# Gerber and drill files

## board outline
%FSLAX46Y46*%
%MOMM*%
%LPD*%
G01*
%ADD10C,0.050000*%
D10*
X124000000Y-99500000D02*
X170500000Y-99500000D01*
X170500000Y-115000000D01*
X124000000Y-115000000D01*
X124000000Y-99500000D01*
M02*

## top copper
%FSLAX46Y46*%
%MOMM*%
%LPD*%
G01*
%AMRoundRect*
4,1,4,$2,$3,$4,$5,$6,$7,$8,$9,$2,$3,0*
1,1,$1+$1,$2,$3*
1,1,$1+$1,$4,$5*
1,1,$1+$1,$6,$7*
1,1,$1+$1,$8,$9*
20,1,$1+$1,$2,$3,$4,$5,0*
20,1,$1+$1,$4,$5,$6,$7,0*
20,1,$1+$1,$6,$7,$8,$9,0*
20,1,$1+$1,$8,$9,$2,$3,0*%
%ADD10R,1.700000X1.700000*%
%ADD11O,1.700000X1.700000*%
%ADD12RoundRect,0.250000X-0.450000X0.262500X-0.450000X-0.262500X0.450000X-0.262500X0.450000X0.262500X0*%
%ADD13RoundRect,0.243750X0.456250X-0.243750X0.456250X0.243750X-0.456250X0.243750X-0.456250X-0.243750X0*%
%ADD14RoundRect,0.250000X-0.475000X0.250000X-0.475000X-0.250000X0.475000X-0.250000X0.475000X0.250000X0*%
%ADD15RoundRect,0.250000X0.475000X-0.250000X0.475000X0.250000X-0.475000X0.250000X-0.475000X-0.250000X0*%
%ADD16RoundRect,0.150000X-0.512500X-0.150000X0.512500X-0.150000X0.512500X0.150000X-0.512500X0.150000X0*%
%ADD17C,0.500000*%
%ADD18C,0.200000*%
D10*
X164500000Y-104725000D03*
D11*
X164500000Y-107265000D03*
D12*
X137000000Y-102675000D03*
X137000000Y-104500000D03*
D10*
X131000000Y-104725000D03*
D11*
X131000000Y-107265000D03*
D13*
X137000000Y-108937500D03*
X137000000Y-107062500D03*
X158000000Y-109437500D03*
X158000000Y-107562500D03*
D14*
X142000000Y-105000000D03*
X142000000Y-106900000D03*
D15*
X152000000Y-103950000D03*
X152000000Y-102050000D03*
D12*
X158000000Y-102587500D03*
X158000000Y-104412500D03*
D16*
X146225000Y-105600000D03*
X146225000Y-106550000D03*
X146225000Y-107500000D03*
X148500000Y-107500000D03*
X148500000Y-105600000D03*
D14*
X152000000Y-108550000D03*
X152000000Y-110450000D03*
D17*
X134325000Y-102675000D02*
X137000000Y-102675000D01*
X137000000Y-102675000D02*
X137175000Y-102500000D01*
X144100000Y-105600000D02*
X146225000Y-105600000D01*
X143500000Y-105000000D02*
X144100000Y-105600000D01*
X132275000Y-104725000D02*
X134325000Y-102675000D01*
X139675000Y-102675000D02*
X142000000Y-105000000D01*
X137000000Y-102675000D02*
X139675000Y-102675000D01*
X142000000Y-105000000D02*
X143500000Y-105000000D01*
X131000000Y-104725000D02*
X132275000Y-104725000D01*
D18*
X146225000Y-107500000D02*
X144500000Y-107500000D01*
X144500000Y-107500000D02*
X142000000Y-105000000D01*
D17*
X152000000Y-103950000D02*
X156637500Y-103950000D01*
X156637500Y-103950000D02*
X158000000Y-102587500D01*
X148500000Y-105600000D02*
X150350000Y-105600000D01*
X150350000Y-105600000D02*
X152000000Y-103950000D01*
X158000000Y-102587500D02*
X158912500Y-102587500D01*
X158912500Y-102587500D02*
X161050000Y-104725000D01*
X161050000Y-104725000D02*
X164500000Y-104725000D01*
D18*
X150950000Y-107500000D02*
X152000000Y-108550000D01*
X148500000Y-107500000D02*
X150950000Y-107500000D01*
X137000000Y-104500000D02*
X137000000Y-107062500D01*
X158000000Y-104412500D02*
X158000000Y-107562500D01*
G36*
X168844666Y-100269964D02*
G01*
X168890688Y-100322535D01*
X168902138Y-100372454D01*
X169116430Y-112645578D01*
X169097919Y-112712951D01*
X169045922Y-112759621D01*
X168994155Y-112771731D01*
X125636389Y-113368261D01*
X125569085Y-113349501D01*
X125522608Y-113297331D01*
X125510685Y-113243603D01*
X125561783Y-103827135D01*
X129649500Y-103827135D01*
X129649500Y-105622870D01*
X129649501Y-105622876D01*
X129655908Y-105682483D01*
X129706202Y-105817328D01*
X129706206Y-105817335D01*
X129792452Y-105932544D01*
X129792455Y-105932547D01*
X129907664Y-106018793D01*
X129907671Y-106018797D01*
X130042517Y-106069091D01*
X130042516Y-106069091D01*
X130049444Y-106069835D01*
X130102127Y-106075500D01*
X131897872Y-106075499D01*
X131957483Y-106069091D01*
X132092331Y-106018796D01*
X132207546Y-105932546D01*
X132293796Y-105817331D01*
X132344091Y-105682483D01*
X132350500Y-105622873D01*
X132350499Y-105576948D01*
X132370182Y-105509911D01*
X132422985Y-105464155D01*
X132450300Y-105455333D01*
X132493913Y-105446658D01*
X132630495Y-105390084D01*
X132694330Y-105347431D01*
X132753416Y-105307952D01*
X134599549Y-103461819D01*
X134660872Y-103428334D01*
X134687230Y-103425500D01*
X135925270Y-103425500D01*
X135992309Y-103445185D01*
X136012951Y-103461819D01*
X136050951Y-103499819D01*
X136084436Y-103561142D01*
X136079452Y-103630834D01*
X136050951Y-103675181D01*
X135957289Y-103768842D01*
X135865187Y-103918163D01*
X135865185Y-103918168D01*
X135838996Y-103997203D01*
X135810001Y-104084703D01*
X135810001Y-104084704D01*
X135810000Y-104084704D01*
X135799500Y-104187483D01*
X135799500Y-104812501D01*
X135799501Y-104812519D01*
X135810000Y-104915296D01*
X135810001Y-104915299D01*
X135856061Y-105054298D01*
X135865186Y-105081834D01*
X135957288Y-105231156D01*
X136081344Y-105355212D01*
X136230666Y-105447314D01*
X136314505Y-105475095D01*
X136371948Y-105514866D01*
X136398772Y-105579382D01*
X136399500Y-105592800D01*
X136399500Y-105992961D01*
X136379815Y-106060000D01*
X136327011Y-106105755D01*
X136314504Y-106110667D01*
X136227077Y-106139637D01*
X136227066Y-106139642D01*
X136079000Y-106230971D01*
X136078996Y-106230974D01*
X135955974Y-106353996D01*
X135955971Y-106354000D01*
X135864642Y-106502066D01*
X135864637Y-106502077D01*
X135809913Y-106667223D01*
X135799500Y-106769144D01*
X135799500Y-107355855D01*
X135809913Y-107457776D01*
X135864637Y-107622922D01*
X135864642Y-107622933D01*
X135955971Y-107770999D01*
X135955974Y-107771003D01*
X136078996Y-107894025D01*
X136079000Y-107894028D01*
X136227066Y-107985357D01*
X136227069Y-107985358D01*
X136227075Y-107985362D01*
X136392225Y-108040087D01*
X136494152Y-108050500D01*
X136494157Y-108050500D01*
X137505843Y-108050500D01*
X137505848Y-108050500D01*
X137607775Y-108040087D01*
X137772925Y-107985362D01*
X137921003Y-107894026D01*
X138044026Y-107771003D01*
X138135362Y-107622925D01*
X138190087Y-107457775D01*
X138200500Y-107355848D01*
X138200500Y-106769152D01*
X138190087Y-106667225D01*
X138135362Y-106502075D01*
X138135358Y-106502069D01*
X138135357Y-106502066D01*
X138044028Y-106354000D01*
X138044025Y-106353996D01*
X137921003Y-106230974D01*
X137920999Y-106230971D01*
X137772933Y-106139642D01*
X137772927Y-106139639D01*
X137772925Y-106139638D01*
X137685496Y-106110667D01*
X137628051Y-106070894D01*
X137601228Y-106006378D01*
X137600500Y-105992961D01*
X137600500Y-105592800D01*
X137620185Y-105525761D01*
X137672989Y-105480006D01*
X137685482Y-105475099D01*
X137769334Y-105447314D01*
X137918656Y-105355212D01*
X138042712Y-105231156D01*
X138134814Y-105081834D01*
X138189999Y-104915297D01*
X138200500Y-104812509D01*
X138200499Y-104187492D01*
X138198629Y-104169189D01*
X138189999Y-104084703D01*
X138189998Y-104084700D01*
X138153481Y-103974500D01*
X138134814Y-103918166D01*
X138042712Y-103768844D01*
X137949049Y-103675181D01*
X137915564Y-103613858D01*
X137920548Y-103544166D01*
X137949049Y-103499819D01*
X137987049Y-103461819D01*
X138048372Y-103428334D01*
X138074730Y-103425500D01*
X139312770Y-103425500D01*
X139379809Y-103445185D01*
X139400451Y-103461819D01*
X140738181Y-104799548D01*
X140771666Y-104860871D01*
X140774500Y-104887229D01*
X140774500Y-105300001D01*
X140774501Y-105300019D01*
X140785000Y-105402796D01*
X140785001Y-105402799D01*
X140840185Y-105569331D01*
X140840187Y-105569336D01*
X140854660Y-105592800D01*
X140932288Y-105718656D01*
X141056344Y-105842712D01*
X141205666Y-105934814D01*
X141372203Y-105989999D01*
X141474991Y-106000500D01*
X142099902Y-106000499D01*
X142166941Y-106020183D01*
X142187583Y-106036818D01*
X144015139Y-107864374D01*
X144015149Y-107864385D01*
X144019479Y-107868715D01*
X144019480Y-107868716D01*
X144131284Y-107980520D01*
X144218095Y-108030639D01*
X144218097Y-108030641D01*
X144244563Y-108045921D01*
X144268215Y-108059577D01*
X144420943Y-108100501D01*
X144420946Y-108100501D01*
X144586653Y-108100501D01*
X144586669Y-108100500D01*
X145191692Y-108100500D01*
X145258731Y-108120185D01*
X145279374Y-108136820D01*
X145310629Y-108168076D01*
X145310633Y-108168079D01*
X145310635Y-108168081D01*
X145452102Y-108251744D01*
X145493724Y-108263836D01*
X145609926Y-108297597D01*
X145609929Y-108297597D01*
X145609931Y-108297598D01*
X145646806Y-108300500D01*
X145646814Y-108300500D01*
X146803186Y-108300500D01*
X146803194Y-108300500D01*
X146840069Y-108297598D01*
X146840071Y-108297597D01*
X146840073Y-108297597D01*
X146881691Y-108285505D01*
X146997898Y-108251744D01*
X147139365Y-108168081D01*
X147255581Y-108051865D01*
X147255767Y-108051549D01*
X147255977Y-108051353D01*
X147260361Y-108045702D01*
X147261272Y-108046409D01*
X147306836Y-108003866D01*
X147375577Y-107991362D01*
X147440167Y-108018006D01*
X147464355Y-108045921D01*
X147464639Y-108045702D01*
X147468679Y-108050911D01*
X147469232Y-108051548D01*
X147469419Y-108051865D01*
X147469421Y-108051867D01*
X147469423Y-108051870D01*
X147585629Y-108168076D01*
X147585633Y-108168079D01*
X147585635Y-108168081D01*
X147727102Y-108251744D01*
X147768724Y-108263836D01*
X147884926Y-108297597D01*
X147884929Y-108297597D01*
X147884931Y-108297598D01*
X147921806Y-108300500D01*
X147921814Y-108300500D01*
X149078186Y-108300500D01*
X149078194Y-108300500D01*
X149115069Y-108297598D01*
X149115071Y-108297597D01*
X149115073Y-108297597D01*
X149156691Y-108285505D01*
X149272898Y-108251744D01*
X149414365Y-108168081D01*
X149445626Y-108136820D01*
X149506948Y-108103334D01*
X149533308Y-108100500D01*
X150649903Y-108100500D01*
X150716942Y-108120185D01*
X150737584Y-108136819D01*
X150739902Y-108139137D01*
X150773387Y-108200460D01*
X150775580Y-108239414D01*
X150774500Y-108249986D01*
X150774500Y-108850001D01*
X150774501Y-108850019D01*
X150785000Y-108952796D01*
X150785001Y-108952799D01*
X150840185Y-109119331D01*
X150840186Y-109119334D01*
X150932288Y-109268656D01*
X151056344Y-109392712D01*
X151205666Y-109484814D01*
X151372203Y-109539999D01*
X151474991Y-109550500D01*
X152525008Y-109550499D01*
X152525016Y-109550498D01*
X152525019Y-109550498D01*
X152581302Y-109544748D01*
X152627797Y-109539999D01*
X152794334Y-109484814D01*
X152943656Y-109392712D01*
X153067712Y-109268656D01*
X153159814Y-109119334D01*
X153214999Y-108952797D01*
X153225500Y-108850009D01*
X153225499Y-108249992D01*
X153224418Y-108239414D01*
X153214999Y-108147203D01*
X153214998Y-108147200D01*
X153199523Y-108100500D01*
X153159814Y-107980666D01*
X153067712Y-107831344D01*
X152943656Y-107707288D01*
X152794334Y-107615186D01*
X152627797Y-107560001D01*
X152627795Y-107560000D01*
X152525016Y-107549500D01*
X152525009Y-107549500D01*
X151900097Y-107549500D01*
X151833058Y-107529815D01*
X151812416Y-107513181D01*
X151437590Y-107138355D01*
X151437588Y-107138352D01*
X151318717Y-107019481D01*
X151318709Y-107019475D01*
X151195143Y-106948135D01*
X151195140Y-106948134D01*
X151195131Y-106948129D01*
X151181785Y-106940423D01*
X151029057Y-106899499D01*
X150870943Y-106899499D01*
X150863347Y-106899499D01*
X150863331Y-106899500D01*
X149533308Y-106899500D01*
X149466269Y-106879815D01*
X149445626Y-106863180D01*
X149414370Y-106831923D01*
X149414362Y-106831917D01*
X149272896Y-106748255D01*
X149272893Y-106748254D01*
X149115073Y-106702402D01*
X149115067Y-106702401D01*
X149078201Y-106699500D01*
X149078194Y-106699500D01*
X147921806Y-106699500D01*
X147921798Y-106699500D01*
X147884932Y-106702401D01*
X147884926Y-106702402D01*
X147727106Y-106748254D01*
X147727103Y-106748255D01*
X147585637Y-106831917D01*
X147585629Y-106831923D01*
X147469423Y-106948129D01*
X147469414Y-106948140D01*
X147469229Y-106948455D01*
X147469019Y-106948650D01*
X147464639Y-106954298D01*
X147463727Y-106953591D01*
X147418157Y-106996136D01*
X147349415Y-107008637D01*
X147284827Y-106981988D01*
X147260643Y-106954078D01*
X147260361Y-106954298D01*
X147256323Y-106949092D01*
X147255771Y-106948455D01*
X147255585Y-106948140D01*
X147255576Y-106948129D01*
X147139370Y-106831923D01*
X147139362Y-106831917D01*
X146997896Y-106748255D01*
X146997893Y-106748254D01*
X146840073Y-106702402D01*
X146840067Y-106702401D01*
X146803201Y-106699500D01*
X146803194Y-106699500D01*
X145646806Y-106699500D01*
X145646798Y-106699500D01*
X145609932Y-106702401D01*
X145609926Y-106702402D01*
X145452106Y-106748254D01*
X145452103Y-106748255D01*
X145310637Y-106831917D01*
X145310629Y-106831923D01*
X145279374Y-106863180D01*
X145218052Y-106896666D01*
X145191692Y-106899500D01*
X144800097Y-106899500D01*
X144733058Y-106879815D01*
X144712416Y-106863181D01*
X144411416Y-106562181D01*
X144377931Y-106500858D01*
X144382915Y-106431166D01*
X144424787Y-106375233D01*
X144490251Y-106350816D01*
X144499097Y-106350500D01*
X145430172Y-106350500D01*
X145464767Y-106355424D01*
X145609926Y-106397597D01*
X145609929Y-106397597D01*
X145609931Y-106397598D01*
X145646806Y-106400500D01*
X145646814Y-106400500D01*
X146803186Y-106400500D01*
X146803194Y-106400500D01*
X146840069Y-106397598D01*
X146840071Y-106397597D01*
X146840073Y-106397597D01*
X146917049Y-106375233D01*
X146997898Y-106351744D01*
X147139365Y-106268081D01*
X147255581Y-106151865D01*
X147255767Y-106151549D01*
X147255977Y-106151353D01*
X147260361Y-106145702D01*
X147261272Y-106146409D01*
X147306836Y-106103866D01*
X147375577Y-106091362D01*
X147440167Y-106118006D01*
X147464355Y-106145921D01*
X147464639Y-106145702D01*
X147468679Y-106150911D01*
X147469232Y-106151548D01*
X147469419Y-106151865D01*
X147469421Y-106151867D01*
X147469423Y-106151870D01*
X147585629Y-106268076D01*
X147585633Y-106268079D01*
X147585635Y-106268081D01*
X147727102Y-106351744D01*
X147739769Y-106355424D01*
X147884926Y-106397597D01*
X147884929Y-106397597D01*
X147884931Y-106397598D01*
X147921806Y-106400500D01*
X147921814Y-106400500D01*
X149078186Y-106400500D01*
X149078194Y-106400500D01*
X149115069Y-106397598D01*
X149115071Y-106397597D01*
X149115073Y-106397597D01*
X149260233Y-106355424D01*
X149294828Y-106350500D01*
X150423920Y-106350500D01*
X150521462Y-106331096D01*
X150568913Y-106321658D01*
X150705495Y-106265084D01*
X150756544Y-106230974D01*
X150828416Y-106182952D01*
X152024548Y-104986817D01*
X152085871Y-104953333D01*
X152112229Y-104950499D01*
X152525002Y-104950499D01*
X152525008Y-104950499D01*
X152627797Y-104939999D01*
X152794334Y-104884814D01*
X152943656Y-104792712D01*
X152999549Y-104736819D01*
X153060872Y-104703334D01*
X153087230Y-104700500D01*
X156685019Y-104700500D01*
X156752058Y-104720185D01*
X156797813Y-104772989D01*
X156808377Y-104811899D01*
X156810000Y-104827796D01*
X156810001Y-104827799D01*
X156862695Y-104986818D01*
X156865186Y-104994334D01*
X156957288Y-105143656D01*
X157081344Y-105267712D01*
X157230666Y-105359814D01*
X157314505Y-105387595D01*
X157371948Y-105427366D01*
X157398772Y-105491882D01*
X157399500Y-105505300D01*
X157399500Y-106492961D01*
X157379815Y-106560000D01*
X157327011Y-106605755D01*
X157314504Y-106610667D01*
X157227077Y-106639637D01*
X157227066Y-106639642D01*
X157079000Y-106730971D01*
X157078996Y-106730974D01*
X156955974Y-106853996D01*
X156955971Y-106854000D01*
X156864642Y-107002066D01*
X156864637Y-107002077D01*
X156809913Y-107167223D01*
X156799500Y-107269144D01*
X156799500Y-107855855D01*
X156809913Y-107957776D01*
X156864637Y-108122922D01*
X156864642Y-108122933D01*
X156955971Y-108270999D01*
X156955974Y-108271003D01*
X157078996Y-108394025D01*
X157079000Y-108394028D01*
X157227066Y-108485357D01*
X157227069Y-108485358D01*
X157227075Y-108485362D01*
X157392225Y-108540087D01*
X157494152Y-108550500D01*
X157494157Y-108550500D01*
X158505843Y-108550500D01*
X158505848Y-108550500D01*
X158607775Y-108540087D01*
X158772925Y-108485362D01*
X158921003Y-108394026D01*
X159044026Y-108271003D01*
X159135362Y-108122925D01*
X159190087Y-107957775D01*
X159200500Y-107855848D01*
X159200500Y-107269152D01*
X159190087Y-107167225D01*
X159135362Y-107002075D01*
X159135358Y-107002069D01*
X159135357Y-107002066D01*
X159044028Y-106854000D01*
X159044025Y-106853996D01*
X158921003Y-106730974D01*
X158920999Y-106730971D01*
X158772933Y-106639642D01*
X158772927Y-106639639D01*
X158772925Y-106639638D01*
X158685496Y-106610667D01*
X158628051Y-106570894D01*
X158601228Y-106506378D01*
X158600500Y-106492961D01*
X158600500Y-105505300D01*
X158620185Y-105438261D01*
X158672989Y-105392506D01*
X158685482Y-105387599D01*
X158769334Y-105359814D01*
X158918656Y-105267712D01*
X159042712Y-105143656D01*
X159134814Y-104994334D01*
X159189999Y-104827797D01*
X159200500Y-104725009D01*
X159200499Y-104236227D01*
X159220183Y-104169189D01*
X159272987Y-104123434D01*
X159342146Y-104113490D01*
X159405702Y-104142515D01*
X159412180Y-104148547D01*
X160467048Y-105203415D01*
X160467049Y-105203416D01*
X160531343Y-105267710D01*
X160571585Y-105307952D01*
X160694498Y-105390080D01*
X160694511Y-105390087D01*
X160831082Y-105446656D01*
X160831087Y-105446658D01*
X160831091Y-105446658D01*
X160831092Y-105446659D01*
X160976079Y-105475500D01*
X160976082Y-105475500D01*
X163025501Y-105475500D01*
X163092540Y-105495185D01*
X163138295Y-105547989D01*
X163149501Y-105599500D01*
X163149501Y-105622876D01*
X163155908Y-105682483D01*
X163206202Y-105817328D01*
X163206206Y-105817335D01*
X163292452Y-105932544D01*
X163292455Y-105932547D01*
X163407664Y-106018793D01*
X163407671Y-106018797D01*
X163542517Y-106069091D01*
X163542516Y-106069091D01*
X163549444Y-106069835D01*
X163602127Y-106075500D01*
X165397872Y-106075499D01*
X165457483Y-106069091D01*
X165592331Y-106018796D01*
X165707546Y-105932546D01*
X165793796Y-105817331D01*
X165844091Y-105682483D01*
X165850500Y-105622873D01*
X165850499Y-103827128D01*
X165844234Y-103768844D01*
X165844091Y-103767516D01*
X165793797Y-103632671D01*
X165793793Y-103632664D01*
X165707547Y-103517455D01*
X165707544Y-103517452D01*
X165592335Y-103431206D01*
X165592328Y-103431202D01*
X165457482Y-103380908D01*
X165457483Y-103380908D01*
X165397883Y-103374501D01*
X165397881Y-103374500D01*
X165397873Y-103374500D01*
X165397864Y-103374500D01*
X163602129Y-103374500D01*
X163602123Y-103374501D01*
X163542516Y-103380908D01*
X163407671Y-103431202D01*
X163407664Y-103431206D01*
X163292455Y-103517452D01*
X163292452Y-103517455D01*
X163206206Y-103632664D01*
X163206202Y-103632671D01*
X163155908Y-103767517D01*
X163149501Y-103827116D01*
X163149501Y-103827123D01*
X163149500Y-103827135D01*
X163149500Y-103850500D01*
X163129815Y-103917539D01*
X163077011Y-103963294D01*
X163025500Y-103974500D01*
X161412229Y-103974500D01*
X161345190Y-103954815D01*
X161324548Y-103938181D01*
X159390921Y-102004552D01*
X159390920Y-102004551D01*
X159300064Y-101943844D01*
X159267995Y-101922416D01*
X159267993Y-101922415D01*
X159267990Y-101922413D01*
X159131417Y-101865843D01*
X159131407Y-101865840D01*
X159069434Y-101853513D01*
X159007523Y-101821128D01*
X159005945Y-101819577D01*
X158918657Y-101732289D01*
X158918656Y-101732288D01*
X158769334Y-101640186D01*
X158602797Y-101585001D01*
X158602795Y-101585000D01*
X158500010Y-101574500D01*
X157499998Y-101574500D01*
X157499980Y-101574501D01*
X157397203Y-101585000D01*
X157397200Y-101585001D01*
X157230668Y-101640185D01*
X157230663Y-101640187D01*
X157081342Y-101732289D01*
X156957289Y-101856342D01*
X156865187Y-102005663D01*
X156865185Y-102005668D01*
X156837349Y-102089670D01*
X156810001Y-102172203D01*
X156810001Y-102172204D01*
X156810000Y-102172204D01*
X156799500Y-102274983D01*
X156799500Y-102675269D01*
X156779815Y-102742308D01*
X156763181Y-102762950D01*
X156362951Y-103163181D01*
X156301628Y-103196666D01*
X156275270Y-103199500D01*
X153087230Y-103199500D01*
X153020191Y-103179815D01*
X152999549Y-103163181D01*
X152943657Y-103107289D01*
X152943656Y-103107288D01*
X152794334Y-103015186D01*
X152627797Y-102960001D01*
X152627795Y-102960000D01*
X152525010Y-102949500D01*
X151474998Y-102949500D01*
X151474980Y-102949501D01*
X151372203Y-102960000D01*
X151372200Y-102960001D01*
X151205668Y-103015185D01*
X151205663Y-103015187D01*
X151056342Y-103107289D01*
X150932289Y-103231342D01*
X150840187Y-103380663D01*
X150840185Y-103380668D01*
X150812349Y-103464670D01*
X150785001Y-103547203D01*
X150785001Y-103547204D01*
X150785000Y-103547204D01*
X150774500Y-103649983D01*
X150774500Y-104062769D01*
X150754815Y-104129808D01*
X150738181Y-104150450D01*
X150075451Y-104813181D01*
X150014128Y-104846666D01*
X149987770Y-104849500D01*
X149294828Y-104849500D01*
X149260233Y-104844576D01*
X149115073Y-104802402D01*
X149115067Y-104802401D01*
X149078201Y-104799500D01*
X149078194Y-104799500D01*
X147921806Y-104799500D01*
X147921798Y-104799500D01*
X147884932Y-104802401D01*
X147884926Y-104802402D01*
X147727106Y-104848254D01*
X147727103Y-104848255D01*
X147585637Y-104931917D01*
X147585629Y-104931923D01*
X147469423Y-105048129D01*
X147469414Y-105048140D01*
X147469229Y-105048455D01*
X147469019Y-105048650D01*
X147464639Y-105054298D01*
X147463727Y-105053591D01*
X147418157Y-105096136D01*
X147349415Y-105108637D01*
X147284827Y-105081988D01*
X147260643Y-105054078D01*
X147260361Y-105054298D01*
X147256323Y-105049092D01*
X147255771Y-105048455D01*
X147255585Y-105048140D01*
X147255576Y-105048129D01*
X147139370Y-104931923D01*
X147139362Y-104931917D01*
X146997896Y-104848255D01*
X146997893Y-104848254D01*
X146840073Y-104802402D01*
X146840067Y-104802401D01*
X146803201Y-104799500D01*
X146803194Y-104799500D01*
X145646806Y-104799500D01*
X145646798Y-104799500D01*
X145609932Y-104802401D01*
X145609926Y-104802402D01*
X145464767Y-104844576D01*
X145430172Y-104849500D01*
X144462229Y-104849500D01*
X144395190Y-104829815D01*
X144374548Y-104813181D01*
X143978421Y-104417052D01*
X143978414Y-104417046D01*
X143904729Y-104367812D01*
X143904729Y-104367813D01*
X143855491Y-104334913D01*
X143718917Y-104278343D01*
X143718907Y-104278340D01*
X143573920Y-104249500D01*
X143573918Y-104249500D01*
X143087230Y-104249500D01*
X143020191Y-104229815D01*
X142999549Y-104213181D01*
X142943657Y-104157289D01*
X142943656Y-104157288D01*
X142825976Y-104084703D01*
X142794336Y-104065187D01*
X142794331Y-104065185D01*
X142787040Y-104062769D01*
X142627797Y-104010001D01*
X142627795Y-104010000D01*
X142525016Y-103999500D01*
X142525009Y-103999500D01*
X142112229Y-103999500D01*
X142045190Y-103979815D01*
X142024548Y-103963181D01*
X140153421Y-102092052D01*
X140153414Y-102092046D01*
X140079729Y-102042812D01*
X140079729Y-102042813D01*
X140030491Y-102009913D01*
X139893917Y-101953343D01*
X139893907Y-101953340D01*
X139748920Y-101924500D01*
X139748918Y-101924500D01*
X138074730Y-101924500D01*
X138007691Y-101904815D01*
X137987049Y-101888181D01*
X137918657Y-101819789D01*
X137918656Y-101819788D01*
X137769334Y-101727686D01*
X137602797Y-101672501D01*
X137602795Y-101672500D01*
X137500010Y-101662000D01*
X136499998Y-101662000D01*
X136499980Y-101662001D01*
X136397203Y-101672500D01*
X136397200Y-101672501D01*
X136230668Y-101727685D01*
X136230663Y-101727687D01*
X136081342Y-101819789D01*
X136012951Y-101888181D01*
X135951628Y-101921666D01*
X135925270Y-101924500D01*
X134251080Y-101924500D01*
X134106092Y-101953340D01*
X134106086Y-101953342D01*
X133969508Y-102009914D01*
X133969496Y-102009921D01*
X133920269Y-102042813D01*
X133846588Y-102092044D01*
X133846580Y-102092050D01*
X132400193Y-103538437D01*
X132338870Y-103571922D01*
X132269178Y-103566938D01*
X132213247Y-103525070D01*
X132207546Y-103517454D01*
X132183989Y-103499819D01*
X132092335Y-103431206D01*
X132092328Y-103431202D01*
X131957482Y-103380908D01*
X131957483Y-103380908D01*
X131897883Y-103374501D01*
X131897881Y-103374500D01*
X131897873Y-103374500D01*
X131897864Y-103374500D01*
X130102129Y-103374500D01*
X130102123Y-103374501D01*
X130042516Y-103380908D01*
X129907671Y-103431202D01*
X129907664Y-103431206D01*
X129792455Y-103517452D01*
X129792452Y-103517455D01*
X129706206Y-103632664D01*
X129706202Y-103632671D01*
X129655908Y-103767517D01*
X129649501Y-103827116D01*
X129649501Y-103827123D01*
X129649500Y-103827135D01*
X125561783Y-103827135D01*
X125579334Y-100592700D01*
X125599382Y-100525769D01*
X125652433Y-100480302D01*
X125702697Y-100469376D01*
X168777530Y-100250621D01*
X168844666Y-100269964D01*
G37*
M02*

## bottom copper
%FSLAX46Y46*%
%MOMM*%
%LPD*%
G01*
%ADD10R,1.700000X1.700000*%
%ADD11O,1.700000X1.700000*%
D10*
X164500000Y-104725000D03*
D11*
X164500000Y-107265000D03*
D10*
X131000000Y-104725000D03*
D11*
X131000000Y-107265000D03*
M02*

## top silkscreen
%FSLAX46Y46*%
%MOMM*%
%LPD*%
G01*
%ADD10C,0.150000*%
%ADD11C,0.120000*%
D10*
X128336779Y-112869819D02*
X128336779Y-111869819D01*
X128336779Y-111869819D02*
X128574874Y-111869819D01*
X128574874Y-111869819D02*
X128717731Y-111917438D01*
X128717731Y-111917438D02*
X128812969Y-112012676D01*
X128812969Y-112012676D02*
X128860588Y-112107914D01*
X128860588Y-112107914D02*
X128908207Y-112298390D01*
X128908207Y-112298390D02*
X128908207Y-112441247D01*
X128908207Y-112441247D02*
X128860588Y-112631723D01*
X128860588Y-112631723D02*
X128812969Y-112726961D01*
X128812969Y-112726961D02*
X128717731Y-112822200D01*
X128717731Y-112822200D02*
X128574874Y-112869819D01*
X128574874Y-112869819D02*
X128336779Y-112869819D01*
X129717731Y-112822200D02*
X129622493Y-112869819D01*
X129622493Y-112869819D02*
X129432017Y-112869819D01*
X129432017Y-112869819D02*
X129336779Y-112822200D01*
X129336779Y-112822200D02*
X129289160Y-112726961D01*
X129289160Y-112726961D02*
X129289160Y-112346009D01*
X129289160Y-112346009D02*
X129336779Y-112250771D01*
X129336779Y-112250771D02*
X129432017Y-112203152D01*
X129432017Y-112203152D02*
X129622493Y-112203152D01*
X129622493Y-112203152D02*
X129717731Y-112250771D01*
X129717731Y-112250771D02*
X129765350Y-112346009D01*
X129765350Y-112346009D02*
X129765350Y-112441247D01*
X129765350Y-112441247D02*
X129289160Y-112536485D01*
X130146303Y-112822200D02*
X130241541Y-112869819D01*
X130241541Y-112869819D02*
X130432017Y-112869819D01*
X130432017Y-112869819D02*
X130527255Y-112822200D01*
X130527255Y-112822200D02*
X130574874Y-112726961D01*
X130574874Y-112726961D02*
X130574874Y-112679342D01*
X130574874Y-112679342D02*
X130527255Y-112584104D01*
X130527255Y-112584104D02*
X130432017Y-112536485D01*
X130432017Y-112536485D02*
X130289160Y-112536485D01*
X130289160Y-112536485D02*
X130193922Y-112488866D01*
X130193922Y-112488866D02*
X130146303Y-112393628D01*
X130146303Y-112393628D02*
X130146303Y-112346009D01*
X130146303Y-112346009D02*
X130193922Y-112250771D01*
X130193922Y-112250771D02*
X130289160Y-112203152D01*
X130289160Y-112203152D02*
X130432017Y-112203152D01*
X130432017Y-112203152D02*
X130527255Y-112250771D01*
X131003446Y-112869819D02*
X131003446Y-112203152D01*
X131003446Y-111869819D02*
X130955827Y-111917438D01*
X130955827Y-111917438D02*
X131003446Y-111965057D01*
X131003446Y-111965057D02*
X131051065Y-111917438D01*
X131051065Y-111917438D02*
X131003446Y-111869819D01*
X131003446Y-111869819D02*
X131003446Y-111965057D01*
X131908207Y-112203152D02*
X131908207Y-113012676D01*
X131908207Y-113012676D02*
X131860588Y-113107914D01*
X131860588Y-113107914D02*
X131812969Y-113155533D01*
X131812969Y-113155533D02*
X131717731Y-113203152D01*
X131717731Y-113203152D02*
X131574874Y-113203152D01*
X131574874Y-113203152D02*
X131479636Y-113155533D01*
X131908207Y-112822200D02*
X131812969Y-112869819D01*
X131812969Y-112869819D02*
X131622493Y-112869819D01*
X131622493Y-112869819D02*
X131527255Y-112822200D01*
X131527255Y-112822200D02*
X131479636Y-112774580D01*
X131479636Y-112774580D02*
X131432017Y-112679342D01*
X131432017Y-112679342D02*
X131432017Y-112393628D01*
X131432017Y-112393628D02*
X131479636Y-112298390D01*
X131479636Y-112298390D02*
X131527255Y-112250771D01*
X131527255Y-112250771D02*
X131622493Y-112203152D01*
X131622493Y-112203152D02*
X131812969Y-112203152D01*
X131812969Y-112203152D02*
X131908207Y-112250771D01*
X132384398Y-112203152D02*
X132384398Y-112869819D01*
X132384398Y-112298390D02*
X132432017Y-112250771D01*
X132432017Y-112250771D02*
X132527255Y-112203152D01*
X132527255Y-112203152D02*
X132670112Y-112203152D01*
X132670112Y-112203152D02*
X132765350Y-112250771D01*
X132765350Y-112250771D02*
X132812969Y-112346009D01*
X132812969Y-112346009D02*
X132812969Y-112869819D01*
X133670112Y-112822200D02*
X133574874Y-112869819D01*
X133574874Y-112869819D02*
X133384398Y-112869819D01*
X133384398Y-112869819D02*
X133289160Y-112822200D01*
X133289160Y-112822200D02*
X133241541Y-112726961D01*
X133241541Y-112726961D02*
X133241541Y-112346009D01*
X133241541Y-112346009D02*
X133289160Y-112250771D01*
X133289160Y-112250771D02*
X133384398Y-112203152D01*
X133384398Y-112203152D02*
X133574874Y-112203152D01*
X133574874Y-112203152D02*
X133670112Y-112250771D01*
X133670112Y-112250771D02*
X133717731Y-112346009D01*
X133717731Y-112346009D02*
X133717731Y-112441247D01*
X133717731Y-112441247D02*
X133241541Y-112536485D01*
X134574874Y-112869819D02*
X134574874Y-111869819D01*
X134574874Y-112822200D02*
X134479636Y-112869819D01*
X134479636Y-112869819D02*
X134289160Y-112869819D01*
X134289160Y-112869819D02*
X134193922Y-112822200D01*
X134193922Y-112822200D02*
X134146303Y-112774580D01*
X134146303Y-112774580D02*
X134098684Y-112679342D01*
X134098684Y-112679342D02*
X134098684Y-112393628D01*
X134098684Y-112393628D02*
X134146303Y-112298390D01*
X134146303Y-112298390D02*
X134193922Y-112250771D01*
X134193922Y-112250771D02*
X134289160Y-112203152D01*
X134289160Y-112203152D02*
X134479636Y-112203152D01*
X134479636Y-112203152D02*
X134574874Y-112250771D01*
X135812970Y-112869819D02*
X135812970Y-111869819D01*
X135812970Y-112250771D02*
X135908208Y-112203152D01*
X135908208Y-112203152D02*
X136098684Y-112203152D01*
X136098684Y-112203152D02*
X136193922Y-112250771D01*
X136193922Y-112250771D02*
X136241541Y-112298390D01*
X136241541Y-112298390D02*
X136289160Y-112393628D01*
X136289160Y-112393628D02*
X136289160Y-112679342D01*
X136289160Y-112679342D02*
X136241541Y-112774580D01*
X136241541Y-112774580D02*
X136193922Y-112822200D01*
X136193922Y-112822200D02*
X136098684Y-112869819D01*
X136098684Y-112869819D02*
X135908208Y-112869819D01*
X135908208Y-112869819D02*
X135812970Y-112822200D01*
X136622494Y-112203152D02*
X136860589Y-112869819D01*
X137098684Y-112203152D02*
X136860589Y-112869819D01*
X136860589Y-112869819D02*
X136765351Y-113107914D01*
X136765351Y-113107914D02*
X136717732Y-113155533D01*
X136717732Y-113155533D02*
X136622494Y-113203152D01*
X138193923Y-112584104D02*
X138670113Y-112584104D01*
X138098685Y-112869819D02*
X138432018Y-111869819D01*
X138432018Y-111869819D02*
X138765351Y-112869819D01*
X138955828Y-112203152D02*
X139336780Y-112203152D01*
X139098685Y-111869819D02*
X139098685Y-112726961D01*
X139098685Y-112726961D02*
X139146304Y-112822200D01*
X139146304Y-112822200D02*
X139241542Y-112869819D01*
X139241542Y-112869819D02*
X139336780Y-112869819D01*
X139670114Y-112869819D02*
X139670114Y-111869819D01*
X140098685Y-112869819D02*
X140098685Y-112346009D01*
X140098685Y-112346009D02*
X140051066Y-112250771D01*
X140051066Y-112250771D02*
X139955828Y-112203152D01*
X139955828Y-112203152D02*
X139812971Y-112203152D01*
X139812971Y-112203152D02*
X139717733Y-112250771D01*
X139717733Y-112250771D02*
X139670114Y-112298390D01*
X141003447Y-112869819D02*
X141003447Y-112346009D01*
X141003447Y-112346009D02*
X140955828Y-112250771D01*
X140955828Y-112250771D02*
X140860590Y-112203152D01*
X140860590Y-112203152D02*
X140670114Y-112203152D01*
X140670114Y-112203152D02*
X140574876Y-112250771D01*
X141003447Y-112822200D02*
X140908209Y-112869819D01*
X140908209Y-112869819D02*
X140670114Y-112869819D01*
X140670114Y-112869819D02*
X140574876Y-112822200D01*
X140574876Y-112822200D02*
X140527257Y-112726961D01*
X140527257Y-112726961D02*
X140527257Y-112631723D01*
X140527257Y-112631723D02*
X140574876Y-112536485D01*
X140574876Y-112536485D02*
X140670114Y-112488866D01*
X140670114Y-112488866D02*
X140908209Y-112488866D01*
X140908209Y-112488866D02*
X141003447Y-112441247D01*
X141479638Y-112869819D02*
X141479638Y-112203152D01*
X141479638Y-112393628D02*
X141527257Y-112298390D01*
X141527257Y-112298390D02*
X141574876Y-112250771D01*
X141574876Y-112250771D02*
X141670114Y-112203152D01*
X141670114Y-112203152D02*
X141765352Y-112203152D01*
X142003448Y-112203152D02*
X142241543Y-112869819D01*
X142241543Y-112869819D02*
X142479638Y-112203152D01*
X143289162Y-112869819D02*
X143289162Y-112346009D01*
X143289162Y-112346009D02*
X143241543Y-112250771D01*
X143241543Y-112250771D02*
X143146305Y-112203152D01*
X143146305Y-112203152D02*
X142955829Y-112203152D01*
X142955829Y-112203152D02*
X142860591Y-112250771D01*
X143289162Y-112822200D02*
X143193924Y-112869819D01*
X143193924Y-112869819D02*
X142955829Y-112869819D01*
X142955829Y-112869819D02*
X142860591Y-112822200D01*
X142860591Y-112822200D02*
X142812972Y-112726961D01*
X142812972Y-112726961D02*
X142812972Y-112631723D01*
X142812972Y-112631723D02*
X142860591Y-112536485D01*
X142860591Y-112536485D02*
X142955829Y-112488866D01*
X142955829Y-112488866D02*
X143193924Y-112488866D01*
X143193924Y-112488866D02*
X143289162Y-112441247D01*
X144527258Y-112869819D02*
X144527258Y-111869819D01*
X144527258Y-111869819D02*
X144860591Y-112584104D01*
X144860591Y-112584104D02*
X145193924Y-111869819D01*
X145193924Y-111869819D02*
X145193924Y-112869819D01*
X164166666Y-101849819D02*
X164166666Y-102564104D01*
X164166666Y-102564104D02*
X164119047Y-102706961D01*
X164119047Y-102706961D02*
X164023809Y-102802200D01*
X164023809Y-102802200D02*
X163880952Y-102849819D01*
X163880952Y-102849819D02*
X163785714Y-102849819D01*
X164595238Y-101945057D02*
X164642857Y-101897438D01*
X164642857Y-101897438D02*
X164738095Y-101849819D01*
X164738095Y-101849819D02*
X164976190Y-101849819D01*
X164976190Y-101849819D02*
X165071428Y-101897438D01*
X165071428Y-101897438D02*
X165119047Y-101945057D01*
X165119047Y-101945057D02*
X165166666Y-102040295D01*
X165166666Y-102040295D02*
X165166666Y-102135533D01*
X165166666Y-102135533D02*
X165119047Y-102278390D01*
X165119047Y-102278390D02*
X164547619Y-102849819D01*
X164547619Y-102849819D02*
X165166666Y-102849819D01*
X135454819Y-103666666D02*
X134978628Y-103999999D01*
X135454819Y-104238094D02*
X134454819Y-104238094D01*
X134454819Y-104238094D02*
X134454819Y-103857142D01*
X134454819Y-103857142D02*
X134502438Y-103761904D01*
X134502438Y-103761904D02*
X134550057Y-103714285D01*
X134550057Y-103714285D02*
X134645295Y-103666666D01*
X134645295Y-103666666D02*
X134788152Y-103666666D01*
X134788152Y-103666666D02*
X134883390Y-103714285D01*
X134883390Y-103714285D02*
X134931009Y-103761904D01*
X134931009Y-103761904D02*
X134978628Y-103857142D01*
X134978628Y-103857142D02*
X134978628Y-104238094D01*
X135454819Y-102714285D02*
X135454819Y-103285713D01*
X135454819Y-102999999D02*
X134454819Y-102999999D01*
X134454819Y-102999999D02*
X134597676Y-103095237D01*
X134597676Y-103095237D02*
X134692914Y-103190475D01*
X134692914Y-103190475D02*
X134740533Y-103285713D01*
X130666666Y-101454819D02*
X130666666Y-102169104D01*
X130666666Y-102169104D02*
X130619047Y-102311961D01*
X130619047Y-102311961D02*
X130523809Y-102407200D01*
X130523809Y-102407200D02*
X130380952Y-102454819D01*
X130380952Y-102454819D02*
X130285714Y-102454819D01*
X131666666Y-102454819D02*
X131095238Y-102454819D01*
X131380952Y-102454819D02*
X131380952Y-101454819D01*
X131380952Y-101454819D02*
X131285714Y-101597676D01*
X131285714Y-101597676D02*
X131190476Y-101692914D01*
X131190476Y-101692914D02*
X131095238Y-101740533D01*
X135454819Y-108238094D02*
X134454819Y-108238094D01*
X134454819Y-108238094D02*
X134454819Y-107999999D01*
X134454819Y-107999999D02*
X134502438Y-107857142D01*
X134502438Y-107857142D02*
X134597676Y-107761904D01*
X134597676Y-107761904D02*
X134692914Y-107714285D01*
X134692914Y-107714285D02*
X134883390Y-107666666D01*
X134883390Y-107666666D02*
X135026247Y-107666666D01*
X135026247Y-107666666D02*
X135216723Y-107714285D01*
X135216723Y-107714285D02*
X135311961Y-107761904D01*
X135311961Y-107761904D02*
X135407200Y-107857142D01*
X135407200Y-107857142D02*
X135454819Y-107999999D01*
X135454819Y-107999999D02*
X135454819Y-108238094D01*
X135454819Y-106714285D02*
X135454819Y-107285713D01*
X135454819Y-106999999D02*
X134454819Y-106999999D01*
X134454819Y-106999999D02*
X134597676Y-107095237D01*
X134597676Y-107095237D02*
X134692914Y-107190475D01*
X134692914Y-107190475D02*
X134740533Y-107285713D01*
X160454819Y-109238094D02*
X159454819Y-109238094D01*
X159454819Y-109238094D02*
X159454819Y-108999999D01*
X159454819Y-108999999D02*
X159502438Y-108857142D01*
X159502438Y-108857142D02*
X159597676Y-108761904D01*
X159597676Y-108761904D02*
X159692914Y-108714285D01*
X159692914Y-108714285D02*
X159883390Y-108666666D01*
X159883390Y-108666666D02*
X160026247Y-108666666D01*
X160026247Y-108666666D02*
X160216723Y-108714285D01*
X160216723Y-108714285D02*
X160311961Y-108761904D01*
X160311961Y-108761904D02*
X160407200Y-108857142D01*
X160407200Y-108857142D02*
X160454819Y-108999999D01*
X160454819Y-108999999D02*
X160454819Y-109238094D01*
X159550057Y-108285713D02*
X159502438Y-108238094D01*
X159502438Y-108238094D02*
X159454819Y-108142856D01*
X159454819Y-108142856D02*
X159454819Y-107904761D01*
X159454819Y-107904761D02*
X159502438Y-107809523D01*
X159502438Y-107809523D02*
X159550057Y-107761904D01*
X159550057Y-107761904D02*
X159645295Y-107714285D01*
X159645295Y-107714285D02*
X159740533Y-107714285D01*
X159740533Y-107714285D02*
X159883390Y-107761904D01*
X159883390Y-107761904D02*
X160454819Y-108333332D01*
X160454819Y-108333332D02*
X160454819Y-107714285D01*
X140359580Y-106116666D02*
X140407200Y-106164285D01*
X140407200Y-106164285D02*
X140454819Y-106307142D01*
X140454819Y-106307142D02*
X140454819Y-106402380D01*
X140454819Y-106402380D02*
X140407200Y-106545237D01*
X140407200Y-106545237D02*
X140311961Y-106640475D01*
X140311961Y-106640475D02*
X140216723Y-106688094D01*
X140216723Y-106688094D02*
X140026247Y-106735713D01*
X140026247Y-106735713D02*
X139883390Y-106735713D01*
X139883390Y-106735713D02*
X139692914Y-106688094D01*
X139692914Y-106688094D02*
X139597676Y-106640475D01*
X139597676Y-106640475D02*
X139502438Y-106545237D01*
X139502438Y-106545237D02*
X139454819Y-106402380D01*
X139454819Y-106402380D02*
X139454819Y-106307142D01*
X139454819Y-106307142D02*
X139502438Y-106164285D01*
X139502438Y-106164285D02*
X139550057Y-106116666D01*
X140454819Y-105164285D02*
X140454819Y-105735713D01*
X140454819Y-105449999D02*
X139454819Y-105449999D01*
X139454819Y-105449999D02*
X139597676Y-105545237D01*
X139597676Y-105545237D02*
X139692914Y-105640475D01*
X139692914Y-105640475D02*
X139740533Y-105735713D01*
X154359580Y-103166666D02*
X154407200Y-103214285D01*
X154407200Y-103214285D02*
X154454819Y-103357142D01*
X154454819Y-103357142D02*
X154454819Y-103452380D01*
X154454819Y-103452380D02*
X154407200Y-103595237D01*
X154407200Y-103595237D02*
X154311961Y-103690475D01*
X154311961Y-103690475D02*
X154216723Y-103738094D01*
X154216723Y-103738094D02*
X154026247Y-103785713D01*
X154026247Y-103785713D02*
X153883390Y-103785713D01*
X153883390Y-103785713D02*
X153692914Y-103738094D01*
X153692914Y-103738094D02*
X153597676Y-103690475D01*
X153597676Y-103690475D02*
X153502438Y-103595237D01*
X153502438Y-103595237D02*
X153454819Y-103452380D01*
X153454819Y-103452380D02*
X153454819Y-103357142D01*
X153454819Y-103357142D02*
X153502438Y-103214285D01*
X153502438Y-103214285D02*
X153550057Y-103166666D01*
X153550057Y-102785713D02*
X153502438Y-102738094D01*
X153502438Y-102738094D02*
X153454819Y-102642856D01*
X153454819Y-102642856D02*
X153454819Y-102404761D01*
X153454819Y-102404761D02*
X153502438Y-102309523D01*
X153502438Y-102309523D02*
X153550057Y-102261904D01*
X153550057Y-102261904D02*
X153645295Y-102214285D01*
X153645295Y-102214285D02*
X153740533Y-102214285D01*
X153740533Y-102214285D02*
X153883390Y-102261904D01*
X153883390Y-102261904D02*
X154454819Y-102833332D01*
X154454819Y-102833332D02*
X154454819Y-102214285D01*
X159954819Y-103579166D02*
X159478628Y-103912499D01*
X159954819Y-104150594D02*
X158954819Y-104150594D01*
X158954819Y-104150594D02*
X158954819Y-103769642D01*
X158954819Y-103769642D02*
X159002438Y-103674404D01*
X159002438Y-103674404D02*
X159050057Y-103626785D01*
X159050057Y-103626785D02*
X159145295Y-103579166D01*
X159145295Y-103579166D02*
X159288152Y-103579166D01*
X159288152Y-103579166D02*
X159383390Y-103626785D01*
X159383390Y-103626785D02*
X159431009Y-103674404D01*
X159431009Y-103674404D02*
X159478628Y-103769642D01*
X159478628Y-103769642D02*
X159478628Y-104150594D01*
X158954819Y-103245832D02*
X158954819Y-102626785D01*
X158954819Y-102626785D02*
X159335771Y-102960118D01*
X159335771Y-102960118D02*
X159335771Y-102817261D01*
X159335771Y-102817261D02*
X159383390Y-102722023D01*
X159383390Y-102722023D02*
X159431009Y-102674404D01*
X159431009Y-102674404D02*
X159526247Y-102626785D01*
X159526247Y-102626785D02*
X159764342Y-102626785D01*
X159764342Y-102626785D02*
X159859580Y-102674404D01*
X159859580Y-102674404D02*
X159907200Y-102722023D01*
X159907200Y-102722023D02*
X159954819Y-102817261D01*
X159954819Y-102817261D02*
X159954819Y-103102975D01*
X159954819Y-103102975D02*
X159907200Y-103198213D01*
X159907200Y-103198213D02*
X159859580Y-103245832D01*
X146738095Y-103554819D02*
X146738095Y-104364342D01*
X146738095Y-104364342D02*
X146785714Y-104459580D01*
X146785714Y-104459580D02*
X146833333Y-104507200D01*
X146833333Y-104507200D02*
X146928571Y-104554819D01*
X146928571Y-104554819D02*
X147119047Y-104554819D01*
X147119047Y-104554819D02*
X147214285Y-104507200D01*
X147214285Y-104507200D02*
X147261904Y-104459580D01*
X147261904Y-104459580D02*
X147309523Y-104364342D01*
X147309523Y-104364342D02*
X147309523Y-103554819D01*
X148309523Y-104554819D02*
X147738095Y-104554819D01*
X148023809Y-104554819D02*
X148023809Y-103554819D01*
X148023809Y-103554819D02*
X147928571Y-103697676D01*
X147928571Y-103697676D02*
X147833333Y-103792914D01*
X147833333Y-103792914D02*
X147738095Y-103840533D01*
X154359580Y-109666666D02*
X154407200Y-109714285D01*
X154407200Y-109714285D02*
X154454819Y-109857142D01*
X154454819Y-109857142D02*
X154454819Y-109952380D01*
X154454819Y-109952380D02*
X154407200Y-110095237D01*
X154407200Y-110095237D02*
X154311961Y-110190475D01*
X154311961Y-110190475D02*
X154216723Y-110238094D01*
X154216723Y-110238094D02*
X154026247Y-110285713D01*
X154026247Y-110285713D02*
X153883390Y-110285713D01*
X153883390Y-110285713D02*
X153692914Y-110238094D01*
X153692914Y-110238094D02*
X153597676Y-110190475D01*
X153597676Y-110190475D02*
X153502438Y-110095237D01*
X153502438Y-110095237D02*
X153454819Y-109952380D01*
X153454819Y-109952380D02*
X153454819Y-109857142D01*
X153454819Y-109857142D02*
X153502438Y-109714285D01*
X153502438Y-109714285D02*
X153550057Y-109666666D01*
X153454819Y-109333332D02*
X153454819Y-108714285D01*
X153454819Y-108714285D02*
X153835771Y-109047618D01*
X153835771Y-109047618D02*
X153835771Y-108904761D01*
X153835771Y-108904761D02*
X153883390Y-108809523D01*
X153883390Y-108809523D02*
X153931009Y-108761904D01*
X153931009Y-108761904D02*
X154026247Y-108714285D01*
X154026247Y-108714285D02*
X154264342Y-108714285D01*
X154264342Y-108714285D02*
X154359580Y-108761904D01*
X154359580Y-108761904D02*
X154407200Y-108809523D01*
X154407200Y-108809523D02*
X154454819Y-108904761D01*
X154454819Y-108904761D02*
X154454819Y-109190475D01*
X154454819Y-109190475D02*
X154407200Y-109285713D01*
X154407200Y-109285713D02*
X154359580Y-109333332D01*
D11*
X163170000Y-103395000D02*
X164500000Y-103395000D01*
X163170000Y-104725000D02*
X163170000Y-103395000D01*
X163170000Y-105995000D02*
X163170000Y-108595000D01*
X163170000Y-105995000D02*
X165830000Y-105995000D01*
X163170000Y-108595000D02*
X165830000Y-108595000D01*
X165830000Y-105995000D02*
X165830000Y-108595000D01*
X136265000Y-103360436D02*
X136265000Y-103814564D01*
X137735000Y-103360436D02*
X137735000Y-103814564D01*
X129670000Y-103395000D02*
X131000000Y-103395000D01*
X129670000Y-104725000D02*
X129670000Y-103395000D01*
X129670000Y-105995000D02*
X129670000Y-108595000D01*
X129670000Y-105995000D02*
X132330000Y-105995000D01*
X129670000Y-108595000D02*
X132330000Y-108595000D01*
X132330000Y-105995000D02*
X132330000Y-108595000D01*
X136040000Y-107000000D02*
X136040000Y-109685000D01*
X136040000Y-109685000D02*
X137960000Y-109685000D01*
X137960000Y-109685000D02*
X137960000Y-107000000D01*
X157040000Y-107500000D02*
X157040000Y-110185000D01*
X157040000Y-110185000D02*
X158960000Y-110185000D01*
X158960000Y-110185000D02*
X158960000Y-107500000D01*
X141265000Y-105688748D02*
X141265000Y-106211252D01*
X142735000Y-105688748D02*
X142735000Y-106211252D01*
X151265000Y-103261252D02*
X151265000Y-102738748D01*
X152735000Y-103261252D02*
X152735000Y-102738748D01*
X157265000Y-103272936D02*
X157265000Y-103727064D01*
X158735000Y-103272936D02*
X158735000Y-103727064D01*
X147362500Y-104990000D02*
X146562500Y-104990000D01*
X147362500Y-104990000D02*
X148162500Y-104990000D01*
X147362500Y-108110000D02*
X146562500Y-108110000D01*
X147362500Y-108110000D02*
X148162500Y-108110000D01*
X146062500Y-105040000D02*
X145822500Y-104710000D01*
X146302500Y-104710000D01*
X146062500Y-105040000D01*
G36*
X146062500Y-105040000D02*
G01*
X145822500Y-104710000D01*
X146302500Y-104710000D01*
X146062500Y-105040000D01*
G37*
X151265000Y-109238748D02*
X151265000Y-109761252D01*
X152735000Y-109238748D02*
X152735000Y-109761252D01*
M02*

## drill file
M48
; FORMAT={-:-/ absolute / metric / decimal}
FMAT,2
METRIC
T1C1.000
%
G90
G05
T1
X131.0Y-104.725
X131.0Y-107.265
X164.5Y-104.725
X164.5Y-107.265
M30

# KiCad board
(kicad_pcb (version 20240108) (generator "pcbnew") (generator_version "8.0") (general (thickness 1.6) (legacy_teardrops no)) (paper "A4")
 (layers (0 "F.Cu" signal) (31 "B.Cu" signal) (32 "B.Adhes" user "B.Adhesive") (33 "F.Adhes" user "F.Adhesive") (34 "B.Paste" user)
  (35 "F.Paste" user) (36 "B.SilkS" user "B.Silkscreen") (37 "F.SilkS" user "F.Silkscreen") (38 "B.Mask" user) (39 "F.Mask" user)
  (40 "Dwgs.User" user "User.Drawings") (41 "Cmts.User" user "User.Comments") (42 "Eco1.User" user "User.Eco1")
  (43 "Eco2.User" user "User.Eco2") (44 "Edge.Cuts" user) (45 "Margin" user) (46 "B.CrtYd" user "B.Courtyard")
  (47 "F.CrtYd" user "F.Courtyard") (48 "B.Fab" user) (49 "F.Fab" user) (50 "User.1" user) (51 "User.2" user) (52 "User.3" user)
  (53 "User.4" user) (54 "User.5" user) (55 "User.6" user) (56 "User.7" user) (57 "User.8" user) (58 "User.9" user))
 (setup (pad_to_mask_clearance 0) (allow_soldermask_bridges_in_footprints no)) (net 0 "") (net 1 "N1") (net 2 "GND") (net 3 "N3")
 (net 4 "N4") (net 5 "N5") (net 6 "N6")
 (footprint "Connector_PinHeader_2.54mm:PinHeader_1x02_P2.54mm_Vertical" (layer "F.Cu") (at 164.5 104.725)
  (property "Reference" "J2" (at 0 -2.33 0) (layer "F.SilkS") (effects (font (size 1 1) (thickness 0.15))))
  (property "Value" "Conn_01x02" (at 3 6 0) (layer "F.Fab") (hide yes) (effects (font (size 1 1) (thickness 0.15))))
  (fp_line (start -1.33 -1.33) (end 0 -1.33) (stroke (width 0.12) (type solid)) (layer "F.SilkS"))
  (fp_line (start -1.33 0) (end -1.33 -1.33) (stroke (width 0.12) (type solid)) (layer "F.SilkS"))
  (fp_line (start -1.33 1.27) (end -1.33 3.87) (stroke (width 0.12) (type solid)) (layer "F.SilkS"))
  (fp_line (start -1.33 1.27) (end 1.33 1.27) (stroke (width 0.12) (type solid)) (layer "F.SilkS"))
  (fp_line (start -1.33 3.87) (end 1.33 3.87) (stroke (width 0.12) (type solid)) (layer "F.SilkS"))
  (fp_line (start 1.33 1.27) (end 1.33 3.87) (stroke (width 0.12) (type solid)) (layer "F.SilkS"))
  (pad "1" thru_hole rect (at 0 0) (size 1.7 1.7) (drill 1) (layers "*.Cu" "*.Mask") (remove_unused_layers no) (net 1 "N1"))
  (pad "2" thru_hole oval (at 0 2.54) (size 1.7 1.7) (drill 1) (layers "*.Cu" "*.Mask") (remove_unused_layers no) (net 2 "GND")))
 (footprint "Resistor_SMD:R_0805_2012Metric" (layer "F.Cu") (at 137 103.5875 -90)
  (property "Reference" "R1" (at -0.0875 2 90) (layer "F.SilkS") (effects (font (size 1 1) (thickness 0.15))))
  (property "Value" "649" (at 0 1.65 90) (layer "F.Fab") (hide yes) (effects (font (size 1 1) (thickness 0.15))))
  (fp_line (start -0.227064 0.735) (end 0.227064 0.735) (stroke (width 0.12) (type solid)) (layer "F.SilkS"))
  (fp_line (start -0.227064 -0.735) (end 0.227064 -0.735) (stroke (width 0.12) (type solid)) (layer "F.SilkS"))
  (pad "1" smd roundrect (at -0.9125 0 270) (size 1.025 1.4) (layers "F.Cu" "F.Paste" "F.Mask") (roundrect_rratio 0.243902) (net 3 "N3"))
  (pad "2" smd roundrect (at 0.9125 0 270) (size 1.025 1.4) (layers "F.Cu" "F.Paste" "F.Mask") (roundrect_rratio 0.243902) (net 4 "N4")))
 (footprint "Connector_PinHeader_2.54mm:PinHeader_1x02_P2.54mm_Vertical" (layer "F.Cu") (at 131 104.725)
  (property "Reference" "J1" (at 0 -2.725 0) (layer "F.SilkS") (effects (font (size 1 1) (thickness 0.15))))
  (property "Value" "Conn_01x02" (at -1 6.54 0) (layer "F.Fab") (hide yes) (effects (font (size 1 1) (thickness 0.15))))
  (fp_line (start -1.33 -1.33) (end 0 -1.33) (stroke (width 0.12) (type solid)) (layer "F.SilkS"))
  (fp_line (start -1.33 0) (end -1.33 -1.33) (stroke (width 0.12) (type solid)) (layer "F.SilkS"))
  (fp_line (start -1.33 1.27) (end -1.33 3.87) (stroke (width 0.12) (type solid)) (layer "F.SilkS"))
  (fp_line (start -1.33 1.27) (end 1.33 1.27) (stroke (width 0.12) (type solid)) (layer "F.SilkS"))
  (fp_line (start -1.33 3.87) (end 1.33 3.87) (stroke (width 0.12) (type solid)) (layer "F.SilkS"))
  (fp_line (start 1.33 1.27) (end 1.33 3.87) (stroke (width 0.12) (type solid)) (layer "F.SilkS"))
  (pad "1" thru_hole rect (at 0 0) (size 1.7 1.7) (drill 1) (layers "*.Cu" "*.Mask") (remove_unused_layers no) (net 3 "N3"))
  (pad "2" thru_hole oval (at 0 2.54) (size 1.7 1.7) (drill 1) (layers "*.Cu" "*.Mask") (remove_unused_layers no) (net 2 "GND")))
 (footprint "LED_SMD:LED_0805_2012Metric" (layer "F.Cu") (at 137 108 90)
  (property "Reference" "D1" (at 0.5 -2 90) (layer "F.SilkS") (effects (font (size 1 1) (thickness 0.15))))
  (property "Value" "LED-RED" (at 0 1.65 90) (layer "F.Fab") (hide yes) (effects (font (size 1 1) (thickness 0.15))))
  (fp_line (start 1 -0.96) (end -1.685 -0.96) (stroke (width 0.12) (type solid)) (layer "F.SilkS"))
  (fp_line (start -1.685 -0.96) (end -1.685 0.96) (stroke (width 0.12) (type solid)) (layer "F.SilkS"))
  (fp_line (start -1.685 0.96) (end 1 0.96) (stroke (width 0.12) (type solid)) (layer "F.SilkS"))
  (pad "1" smd roundrect (at -0.9375 0 90) (size 0.975 1.4) (layers "F.Cu" "F.Paste" "F.Mask") (roundrect_rratio 0.25) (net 2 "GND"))
  (pad "2" smd roundrect (at 0.9375 0 90) (size 0.975 1.4) (layers "F.Cu" "F.Paste" "F.Mask") (roundrect_rratio 0.25) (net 4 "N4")))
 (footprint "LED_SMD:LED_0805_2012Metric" (layer "F.Cu") (at 158 108.5 90)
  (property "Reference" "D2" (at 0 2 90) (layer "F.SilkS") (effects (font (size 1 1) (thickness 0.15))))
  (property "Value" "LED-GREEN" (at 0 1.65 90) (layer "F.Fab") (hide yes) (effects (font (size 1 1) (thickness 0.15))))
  (fp_line (start 1 -0.96) (end -1.685 -0.96) (stroke (width 0.12) (type solid)) (layer "F.SilkS"))
  (fp_line (start -1.685 -0.96) (end -1.685 0.96) (stroke (width 0.12) (type solid)) (layer "F.SilkS"))
  (fp_line (start -1.685 0.96) (end 1 0.96) (stroke (width 0.12) (type solid)) (layer "F.SilkS"))
  (pad "1" smd roundrect (at -0.9375 0 90) (size 0.975 1.4) (layers "F.Cu" "F.Paste" "F.Mask") (roundrect_rratio 0.25) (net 2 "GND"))
  (pad "2" smd roundrect (at 0.9375 0 90) (size 0.975 1.4) (layers "F.Cu" "F.Paste" "F.Mask") (roundrect_rratio 0.25) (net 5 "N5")))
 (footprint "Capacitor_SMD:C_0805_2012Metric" (layer "F.Cu") (at 142 105.95 -90)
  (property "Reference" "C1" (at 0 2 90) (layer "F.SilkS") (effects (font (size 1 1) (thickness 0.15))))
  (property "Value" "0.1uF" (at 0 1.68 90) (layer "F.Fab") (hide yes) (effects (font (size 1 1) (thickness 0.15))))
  (fp_line (start -0.261252 0.735) (end 0.261252 0.735) (stroke (width 0.12) (type solid)) (layer "F.SilkS"))
  (fp_line (start -0.261252 -0.735) (end 0.261252 -0.735) (stroke (width 0.12) (type solid)) (layer "F.SilkS"))
  (pad "1" smd roundrect (at -0.95 0 270) (size 1 1.45) (layers "F.Cu" "F.Paste" "F.Mask") (roundrect_rratio 0.25) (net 3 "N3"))
  (pad "2" smd roundrect (at 0.95 0 270) (size 1 1.45) (layers "F.Cu" "F.Paste" "F.Mask") (roundrect_rratio 0.25) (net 2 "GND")))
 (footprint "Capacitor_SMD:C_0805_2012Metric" (layer "F.Cu") (at 152 103 90)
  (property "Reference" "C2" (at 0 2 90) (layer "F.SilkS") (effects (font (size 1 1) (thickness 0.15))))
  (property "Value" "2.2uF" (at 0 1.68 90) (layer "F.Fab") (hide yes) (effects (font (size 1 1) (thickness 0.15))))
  (fp_line (start -0.261252 -0.735) (end 0.261252 -0.735) (stroke (width 0.12) (type solid)) (layer "F.SilkS"))
  (fp_line (start -0.261252 0.735) (end 0.261252 0.735) (stroke (width 0.12) (type solid)) (layer "F.SilkS"))
  (pad "1" smd roundrect (at -0.95 0 90) (size 1 1.45) (layers "F.Cu" "F.Paste" "F.Mask") (roundrect_rratio 0.25) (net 1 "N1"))
  (pad "2" smd roundrect (at 0.95 0 90) (size 1 1.45) (layers "F.Cu" "F.Paste" "F.Mask") (roundrect_rratio 0.25) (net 2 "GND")))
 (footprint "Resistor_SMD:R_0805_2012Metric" (layer "F.Cu") (at 158 103.5 -90)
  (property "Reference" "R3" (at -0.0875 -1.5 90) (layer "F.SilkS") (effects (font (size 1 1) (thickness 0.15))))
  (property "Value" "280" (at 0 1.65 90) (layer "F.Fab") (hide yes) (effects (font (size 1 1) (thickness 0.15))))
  (fp_line (start -0.227064 0.735) (end 0.227064 0.735) (stroke (width 0.12) (type solid)) (layer "F.SilkS"))
  (fp_line (start -0.227064 -0.735) (end 0.227064 -0.735) (stroke (width 0.12) (type solid)) (layer "F.SilkS"))
  (pad "1" smd roundrect (at -0.9125 0 270) (size 1.025 1.4) (layers "F.Cu" "F.Paste" "F.Mask") (roundrect_rratio 0.243902) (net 1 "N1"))
  (pad "2" smd roundrect (at 0.9125 0 270) (size 1.025 1.4) (layers "F.Cu" "F.Paste" "F.Mask") (roundrect_rratio 0.243902) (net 5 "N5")))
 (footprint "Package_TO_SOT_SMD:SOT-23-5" (layer "F.Cu") (at 147.3625 106.55)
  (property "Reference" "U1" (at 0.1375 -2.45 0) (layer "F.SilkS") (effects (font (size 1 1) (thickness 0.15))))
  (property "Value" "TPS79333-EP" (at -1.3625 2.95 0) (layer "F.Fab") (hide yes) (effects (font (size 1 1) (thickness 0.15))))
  (fp_line (start 0 -1.56) (end -0.8 -1.56) (stroke (width 0.12) (type solid)) (layer "F.SilkS"))
  (fp_line (start 0 -1.56) (end 0.8 -1.56) (stroke (width 0.12) (type solid)) (layer "F.SilkS"))
  (fp_line (start 0 1.56) (end -0.8 1.56) (stroke (width 0.12) (type solid)) (layer "F.SilkS"))
  (fp_line (start 0 1.56) (end 0.8 1.56) (stroke (width 0.12) (type solid)) (layer "F.SilkS"))
  (fp_poly
   (pts (xy -1.3 -1.51) (xy -1.54 -1.84) (xy -1.06 -1.84) (xy -1.3 -1.51)) (stroke (width 0.12) (type solid)) (fill solid) (layer "F.SilkS"))
  (pad "1" smd roundrect (at -1.1375 -0.95) (size 1.325 0.6) (layers "F.Cu" "F.Paste" "F.Mask") (roundrect_rratio 0.25) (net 3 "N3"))
  (pad "2" smd roundrect (at -1.1375 0) (size 1.325 0.6) (layers "F.Cu" "F.Paste" "F.Mask") (roundrect_rratio 0.25) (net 2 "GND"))
  (pad "3" smd roundrect (at -1.1375 0.95) (size 1.325 0.6) (layers "F.Cu" "F.Paste" "F.Mask") (roundrect_rratio 0.25) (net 3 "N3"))
  (pad "4" smd roundrect (at 1.1375 0.95) (size 1.325 0.6) (layers "F.Cu" "F.Paste" "F.Mask") (roundrect_rratio 0.25) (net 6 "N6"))
  (pad "5" smd roundrect (at 1.1375 -0.95) (size 1.325 0.6) (layers "F.Cu" "F.Paste" "F.Mask") (roundrect_rratio 0.25) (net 1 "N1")))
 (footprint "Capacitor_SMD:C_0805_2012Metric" (layer "F.Cu") (at 152 109.5 -90)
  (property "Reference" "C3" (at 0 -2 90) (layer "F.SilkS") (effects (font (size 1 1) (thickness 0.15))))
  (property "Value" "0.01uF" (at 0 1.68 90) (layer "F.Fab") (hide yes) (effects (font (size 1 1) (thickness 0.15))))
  (fp_line (start -0.261252 0.735) (end 0.261252 0.735) (stroke (width 0.12) (type solid)) (layer "F.SilkS"))
  (fp_line (start -0.261252 -0.735) (end 0.261252 -0.735) (stroke (width 0.12) (type solid)) (layer "F.SilkS"))
  (pad "1" smd roundrect (at -0.95 0 270) (size 1 1.45) (layers "F.Cu" "F.Paste" "F.Mask") (roundrect_rratio 0.25) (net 6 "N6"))
  (pad "2" smd roundrect (at 0.95 0 270) (size 1 1.45) (layers "F.Cu" "F.Paste" "F.Mask") (roundrect_rratio 0.25) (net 2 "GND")))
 (gr_rect (start 124 99.5) (end 170.5 115) (stroke (width 0.05) (type default)) (fill none) (layer "Edge.Cuts"))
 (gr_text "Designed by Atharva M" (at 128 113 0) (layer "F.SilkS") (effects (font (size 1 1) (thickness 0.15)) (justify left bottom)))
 (segment (start 134.325 102.675) (end 137 102.675) (width 0.5) (layer "F.Cu") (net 3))
 (segment (start 137 102.675) (end 137.175 102.5) (width 0.5) (layer "F.Cu") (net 3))
 (segment (start 144.1 105.6) (end 146.225 105.6) (width 0.5) (layer "F.Cu") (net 3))
 (segment (start 143.5 105) (end 144.1 105.6) (width 0.5) (layer "F.Cu") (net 3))
 (segment (start 132.275 104.725) (end 134.325 102.675) (width 0.5) (layer "F.Cu") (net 3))
 (segment (start 139.675 102.675) (end 142 105) (width 0.5) (layer "F.Cu") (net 3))
 (segment (start 137 102.675) (end 139.675 102.675) (width 0.5) (layer "F.Cu") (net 3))
 (segment (start 142 105) (end 143.5 105) (width 0.5) (layer "F.Cu") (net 3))
 (segment (start 131 104.725) (end 132.275 104.725) (width 0.5) (layer "F.Cu") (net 3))
 (segment (start 146.225 107.5) (end 144.5 107.5) (width 0.2) (layer "F.Cu") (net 3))
 (segment (start 144.5 107.5) (end 142 105) (width 0.2) (layer "F.Cu") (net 3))
 (segment (start 152 103.95) (end 156.6375 103.95) (width 0.5) (layer "F.Cu") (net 1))
 (segment (start 156.6375 103.95) (end 158 102.5875) (width 0.5) (layer "F.Cu") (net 1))
 (segment (start 148.5 105.6) (end 150.35 105.6) (width 0.5) (layer "F.Cu") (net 1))
 (segment (start 150.35 105.6) (end 152 103.95) (width 0.5) (layer "F.Cu") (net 1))
 (segment (start 158 102.5875) (end 158.9125 102.5875) (width 0.5) (layer "F.Cu") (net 1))
 (segment (start 158.9125 102.5875) (end 161.05 104.725) (width 0.5) (layer "F.Cu") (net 1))
 (segment (start 161.05 104.725) (end 164.5 104.725) (width 0.5) (layer "F.Cu") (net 1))
 (segment (start 150.95 107.5) (end 152 108.55) (width 0.2) (layer "F.Cu") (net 6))
 (segment (start 148.5 107.5) (end 150.95 107.5) (width 0.2) (layer "F.Cu") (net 6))
 (segment (start 137 104.5) (end 137 107.0625) (width 0.2) (layer "F.Cu") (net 4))
 (segment (start 158 104.4125) (end 158 107.5625) (width 0.2) (layer "F.Cu") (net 5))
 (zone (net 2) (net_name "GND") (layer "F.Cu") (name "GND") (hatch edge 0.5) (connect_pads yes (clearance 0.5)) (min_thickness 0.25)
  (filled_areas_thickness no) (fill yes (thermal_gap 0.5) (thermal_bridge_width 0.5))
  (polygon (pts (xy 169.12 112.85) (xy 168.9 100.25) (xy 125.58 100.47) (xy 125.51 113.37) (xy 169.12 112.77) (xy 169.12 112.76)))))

